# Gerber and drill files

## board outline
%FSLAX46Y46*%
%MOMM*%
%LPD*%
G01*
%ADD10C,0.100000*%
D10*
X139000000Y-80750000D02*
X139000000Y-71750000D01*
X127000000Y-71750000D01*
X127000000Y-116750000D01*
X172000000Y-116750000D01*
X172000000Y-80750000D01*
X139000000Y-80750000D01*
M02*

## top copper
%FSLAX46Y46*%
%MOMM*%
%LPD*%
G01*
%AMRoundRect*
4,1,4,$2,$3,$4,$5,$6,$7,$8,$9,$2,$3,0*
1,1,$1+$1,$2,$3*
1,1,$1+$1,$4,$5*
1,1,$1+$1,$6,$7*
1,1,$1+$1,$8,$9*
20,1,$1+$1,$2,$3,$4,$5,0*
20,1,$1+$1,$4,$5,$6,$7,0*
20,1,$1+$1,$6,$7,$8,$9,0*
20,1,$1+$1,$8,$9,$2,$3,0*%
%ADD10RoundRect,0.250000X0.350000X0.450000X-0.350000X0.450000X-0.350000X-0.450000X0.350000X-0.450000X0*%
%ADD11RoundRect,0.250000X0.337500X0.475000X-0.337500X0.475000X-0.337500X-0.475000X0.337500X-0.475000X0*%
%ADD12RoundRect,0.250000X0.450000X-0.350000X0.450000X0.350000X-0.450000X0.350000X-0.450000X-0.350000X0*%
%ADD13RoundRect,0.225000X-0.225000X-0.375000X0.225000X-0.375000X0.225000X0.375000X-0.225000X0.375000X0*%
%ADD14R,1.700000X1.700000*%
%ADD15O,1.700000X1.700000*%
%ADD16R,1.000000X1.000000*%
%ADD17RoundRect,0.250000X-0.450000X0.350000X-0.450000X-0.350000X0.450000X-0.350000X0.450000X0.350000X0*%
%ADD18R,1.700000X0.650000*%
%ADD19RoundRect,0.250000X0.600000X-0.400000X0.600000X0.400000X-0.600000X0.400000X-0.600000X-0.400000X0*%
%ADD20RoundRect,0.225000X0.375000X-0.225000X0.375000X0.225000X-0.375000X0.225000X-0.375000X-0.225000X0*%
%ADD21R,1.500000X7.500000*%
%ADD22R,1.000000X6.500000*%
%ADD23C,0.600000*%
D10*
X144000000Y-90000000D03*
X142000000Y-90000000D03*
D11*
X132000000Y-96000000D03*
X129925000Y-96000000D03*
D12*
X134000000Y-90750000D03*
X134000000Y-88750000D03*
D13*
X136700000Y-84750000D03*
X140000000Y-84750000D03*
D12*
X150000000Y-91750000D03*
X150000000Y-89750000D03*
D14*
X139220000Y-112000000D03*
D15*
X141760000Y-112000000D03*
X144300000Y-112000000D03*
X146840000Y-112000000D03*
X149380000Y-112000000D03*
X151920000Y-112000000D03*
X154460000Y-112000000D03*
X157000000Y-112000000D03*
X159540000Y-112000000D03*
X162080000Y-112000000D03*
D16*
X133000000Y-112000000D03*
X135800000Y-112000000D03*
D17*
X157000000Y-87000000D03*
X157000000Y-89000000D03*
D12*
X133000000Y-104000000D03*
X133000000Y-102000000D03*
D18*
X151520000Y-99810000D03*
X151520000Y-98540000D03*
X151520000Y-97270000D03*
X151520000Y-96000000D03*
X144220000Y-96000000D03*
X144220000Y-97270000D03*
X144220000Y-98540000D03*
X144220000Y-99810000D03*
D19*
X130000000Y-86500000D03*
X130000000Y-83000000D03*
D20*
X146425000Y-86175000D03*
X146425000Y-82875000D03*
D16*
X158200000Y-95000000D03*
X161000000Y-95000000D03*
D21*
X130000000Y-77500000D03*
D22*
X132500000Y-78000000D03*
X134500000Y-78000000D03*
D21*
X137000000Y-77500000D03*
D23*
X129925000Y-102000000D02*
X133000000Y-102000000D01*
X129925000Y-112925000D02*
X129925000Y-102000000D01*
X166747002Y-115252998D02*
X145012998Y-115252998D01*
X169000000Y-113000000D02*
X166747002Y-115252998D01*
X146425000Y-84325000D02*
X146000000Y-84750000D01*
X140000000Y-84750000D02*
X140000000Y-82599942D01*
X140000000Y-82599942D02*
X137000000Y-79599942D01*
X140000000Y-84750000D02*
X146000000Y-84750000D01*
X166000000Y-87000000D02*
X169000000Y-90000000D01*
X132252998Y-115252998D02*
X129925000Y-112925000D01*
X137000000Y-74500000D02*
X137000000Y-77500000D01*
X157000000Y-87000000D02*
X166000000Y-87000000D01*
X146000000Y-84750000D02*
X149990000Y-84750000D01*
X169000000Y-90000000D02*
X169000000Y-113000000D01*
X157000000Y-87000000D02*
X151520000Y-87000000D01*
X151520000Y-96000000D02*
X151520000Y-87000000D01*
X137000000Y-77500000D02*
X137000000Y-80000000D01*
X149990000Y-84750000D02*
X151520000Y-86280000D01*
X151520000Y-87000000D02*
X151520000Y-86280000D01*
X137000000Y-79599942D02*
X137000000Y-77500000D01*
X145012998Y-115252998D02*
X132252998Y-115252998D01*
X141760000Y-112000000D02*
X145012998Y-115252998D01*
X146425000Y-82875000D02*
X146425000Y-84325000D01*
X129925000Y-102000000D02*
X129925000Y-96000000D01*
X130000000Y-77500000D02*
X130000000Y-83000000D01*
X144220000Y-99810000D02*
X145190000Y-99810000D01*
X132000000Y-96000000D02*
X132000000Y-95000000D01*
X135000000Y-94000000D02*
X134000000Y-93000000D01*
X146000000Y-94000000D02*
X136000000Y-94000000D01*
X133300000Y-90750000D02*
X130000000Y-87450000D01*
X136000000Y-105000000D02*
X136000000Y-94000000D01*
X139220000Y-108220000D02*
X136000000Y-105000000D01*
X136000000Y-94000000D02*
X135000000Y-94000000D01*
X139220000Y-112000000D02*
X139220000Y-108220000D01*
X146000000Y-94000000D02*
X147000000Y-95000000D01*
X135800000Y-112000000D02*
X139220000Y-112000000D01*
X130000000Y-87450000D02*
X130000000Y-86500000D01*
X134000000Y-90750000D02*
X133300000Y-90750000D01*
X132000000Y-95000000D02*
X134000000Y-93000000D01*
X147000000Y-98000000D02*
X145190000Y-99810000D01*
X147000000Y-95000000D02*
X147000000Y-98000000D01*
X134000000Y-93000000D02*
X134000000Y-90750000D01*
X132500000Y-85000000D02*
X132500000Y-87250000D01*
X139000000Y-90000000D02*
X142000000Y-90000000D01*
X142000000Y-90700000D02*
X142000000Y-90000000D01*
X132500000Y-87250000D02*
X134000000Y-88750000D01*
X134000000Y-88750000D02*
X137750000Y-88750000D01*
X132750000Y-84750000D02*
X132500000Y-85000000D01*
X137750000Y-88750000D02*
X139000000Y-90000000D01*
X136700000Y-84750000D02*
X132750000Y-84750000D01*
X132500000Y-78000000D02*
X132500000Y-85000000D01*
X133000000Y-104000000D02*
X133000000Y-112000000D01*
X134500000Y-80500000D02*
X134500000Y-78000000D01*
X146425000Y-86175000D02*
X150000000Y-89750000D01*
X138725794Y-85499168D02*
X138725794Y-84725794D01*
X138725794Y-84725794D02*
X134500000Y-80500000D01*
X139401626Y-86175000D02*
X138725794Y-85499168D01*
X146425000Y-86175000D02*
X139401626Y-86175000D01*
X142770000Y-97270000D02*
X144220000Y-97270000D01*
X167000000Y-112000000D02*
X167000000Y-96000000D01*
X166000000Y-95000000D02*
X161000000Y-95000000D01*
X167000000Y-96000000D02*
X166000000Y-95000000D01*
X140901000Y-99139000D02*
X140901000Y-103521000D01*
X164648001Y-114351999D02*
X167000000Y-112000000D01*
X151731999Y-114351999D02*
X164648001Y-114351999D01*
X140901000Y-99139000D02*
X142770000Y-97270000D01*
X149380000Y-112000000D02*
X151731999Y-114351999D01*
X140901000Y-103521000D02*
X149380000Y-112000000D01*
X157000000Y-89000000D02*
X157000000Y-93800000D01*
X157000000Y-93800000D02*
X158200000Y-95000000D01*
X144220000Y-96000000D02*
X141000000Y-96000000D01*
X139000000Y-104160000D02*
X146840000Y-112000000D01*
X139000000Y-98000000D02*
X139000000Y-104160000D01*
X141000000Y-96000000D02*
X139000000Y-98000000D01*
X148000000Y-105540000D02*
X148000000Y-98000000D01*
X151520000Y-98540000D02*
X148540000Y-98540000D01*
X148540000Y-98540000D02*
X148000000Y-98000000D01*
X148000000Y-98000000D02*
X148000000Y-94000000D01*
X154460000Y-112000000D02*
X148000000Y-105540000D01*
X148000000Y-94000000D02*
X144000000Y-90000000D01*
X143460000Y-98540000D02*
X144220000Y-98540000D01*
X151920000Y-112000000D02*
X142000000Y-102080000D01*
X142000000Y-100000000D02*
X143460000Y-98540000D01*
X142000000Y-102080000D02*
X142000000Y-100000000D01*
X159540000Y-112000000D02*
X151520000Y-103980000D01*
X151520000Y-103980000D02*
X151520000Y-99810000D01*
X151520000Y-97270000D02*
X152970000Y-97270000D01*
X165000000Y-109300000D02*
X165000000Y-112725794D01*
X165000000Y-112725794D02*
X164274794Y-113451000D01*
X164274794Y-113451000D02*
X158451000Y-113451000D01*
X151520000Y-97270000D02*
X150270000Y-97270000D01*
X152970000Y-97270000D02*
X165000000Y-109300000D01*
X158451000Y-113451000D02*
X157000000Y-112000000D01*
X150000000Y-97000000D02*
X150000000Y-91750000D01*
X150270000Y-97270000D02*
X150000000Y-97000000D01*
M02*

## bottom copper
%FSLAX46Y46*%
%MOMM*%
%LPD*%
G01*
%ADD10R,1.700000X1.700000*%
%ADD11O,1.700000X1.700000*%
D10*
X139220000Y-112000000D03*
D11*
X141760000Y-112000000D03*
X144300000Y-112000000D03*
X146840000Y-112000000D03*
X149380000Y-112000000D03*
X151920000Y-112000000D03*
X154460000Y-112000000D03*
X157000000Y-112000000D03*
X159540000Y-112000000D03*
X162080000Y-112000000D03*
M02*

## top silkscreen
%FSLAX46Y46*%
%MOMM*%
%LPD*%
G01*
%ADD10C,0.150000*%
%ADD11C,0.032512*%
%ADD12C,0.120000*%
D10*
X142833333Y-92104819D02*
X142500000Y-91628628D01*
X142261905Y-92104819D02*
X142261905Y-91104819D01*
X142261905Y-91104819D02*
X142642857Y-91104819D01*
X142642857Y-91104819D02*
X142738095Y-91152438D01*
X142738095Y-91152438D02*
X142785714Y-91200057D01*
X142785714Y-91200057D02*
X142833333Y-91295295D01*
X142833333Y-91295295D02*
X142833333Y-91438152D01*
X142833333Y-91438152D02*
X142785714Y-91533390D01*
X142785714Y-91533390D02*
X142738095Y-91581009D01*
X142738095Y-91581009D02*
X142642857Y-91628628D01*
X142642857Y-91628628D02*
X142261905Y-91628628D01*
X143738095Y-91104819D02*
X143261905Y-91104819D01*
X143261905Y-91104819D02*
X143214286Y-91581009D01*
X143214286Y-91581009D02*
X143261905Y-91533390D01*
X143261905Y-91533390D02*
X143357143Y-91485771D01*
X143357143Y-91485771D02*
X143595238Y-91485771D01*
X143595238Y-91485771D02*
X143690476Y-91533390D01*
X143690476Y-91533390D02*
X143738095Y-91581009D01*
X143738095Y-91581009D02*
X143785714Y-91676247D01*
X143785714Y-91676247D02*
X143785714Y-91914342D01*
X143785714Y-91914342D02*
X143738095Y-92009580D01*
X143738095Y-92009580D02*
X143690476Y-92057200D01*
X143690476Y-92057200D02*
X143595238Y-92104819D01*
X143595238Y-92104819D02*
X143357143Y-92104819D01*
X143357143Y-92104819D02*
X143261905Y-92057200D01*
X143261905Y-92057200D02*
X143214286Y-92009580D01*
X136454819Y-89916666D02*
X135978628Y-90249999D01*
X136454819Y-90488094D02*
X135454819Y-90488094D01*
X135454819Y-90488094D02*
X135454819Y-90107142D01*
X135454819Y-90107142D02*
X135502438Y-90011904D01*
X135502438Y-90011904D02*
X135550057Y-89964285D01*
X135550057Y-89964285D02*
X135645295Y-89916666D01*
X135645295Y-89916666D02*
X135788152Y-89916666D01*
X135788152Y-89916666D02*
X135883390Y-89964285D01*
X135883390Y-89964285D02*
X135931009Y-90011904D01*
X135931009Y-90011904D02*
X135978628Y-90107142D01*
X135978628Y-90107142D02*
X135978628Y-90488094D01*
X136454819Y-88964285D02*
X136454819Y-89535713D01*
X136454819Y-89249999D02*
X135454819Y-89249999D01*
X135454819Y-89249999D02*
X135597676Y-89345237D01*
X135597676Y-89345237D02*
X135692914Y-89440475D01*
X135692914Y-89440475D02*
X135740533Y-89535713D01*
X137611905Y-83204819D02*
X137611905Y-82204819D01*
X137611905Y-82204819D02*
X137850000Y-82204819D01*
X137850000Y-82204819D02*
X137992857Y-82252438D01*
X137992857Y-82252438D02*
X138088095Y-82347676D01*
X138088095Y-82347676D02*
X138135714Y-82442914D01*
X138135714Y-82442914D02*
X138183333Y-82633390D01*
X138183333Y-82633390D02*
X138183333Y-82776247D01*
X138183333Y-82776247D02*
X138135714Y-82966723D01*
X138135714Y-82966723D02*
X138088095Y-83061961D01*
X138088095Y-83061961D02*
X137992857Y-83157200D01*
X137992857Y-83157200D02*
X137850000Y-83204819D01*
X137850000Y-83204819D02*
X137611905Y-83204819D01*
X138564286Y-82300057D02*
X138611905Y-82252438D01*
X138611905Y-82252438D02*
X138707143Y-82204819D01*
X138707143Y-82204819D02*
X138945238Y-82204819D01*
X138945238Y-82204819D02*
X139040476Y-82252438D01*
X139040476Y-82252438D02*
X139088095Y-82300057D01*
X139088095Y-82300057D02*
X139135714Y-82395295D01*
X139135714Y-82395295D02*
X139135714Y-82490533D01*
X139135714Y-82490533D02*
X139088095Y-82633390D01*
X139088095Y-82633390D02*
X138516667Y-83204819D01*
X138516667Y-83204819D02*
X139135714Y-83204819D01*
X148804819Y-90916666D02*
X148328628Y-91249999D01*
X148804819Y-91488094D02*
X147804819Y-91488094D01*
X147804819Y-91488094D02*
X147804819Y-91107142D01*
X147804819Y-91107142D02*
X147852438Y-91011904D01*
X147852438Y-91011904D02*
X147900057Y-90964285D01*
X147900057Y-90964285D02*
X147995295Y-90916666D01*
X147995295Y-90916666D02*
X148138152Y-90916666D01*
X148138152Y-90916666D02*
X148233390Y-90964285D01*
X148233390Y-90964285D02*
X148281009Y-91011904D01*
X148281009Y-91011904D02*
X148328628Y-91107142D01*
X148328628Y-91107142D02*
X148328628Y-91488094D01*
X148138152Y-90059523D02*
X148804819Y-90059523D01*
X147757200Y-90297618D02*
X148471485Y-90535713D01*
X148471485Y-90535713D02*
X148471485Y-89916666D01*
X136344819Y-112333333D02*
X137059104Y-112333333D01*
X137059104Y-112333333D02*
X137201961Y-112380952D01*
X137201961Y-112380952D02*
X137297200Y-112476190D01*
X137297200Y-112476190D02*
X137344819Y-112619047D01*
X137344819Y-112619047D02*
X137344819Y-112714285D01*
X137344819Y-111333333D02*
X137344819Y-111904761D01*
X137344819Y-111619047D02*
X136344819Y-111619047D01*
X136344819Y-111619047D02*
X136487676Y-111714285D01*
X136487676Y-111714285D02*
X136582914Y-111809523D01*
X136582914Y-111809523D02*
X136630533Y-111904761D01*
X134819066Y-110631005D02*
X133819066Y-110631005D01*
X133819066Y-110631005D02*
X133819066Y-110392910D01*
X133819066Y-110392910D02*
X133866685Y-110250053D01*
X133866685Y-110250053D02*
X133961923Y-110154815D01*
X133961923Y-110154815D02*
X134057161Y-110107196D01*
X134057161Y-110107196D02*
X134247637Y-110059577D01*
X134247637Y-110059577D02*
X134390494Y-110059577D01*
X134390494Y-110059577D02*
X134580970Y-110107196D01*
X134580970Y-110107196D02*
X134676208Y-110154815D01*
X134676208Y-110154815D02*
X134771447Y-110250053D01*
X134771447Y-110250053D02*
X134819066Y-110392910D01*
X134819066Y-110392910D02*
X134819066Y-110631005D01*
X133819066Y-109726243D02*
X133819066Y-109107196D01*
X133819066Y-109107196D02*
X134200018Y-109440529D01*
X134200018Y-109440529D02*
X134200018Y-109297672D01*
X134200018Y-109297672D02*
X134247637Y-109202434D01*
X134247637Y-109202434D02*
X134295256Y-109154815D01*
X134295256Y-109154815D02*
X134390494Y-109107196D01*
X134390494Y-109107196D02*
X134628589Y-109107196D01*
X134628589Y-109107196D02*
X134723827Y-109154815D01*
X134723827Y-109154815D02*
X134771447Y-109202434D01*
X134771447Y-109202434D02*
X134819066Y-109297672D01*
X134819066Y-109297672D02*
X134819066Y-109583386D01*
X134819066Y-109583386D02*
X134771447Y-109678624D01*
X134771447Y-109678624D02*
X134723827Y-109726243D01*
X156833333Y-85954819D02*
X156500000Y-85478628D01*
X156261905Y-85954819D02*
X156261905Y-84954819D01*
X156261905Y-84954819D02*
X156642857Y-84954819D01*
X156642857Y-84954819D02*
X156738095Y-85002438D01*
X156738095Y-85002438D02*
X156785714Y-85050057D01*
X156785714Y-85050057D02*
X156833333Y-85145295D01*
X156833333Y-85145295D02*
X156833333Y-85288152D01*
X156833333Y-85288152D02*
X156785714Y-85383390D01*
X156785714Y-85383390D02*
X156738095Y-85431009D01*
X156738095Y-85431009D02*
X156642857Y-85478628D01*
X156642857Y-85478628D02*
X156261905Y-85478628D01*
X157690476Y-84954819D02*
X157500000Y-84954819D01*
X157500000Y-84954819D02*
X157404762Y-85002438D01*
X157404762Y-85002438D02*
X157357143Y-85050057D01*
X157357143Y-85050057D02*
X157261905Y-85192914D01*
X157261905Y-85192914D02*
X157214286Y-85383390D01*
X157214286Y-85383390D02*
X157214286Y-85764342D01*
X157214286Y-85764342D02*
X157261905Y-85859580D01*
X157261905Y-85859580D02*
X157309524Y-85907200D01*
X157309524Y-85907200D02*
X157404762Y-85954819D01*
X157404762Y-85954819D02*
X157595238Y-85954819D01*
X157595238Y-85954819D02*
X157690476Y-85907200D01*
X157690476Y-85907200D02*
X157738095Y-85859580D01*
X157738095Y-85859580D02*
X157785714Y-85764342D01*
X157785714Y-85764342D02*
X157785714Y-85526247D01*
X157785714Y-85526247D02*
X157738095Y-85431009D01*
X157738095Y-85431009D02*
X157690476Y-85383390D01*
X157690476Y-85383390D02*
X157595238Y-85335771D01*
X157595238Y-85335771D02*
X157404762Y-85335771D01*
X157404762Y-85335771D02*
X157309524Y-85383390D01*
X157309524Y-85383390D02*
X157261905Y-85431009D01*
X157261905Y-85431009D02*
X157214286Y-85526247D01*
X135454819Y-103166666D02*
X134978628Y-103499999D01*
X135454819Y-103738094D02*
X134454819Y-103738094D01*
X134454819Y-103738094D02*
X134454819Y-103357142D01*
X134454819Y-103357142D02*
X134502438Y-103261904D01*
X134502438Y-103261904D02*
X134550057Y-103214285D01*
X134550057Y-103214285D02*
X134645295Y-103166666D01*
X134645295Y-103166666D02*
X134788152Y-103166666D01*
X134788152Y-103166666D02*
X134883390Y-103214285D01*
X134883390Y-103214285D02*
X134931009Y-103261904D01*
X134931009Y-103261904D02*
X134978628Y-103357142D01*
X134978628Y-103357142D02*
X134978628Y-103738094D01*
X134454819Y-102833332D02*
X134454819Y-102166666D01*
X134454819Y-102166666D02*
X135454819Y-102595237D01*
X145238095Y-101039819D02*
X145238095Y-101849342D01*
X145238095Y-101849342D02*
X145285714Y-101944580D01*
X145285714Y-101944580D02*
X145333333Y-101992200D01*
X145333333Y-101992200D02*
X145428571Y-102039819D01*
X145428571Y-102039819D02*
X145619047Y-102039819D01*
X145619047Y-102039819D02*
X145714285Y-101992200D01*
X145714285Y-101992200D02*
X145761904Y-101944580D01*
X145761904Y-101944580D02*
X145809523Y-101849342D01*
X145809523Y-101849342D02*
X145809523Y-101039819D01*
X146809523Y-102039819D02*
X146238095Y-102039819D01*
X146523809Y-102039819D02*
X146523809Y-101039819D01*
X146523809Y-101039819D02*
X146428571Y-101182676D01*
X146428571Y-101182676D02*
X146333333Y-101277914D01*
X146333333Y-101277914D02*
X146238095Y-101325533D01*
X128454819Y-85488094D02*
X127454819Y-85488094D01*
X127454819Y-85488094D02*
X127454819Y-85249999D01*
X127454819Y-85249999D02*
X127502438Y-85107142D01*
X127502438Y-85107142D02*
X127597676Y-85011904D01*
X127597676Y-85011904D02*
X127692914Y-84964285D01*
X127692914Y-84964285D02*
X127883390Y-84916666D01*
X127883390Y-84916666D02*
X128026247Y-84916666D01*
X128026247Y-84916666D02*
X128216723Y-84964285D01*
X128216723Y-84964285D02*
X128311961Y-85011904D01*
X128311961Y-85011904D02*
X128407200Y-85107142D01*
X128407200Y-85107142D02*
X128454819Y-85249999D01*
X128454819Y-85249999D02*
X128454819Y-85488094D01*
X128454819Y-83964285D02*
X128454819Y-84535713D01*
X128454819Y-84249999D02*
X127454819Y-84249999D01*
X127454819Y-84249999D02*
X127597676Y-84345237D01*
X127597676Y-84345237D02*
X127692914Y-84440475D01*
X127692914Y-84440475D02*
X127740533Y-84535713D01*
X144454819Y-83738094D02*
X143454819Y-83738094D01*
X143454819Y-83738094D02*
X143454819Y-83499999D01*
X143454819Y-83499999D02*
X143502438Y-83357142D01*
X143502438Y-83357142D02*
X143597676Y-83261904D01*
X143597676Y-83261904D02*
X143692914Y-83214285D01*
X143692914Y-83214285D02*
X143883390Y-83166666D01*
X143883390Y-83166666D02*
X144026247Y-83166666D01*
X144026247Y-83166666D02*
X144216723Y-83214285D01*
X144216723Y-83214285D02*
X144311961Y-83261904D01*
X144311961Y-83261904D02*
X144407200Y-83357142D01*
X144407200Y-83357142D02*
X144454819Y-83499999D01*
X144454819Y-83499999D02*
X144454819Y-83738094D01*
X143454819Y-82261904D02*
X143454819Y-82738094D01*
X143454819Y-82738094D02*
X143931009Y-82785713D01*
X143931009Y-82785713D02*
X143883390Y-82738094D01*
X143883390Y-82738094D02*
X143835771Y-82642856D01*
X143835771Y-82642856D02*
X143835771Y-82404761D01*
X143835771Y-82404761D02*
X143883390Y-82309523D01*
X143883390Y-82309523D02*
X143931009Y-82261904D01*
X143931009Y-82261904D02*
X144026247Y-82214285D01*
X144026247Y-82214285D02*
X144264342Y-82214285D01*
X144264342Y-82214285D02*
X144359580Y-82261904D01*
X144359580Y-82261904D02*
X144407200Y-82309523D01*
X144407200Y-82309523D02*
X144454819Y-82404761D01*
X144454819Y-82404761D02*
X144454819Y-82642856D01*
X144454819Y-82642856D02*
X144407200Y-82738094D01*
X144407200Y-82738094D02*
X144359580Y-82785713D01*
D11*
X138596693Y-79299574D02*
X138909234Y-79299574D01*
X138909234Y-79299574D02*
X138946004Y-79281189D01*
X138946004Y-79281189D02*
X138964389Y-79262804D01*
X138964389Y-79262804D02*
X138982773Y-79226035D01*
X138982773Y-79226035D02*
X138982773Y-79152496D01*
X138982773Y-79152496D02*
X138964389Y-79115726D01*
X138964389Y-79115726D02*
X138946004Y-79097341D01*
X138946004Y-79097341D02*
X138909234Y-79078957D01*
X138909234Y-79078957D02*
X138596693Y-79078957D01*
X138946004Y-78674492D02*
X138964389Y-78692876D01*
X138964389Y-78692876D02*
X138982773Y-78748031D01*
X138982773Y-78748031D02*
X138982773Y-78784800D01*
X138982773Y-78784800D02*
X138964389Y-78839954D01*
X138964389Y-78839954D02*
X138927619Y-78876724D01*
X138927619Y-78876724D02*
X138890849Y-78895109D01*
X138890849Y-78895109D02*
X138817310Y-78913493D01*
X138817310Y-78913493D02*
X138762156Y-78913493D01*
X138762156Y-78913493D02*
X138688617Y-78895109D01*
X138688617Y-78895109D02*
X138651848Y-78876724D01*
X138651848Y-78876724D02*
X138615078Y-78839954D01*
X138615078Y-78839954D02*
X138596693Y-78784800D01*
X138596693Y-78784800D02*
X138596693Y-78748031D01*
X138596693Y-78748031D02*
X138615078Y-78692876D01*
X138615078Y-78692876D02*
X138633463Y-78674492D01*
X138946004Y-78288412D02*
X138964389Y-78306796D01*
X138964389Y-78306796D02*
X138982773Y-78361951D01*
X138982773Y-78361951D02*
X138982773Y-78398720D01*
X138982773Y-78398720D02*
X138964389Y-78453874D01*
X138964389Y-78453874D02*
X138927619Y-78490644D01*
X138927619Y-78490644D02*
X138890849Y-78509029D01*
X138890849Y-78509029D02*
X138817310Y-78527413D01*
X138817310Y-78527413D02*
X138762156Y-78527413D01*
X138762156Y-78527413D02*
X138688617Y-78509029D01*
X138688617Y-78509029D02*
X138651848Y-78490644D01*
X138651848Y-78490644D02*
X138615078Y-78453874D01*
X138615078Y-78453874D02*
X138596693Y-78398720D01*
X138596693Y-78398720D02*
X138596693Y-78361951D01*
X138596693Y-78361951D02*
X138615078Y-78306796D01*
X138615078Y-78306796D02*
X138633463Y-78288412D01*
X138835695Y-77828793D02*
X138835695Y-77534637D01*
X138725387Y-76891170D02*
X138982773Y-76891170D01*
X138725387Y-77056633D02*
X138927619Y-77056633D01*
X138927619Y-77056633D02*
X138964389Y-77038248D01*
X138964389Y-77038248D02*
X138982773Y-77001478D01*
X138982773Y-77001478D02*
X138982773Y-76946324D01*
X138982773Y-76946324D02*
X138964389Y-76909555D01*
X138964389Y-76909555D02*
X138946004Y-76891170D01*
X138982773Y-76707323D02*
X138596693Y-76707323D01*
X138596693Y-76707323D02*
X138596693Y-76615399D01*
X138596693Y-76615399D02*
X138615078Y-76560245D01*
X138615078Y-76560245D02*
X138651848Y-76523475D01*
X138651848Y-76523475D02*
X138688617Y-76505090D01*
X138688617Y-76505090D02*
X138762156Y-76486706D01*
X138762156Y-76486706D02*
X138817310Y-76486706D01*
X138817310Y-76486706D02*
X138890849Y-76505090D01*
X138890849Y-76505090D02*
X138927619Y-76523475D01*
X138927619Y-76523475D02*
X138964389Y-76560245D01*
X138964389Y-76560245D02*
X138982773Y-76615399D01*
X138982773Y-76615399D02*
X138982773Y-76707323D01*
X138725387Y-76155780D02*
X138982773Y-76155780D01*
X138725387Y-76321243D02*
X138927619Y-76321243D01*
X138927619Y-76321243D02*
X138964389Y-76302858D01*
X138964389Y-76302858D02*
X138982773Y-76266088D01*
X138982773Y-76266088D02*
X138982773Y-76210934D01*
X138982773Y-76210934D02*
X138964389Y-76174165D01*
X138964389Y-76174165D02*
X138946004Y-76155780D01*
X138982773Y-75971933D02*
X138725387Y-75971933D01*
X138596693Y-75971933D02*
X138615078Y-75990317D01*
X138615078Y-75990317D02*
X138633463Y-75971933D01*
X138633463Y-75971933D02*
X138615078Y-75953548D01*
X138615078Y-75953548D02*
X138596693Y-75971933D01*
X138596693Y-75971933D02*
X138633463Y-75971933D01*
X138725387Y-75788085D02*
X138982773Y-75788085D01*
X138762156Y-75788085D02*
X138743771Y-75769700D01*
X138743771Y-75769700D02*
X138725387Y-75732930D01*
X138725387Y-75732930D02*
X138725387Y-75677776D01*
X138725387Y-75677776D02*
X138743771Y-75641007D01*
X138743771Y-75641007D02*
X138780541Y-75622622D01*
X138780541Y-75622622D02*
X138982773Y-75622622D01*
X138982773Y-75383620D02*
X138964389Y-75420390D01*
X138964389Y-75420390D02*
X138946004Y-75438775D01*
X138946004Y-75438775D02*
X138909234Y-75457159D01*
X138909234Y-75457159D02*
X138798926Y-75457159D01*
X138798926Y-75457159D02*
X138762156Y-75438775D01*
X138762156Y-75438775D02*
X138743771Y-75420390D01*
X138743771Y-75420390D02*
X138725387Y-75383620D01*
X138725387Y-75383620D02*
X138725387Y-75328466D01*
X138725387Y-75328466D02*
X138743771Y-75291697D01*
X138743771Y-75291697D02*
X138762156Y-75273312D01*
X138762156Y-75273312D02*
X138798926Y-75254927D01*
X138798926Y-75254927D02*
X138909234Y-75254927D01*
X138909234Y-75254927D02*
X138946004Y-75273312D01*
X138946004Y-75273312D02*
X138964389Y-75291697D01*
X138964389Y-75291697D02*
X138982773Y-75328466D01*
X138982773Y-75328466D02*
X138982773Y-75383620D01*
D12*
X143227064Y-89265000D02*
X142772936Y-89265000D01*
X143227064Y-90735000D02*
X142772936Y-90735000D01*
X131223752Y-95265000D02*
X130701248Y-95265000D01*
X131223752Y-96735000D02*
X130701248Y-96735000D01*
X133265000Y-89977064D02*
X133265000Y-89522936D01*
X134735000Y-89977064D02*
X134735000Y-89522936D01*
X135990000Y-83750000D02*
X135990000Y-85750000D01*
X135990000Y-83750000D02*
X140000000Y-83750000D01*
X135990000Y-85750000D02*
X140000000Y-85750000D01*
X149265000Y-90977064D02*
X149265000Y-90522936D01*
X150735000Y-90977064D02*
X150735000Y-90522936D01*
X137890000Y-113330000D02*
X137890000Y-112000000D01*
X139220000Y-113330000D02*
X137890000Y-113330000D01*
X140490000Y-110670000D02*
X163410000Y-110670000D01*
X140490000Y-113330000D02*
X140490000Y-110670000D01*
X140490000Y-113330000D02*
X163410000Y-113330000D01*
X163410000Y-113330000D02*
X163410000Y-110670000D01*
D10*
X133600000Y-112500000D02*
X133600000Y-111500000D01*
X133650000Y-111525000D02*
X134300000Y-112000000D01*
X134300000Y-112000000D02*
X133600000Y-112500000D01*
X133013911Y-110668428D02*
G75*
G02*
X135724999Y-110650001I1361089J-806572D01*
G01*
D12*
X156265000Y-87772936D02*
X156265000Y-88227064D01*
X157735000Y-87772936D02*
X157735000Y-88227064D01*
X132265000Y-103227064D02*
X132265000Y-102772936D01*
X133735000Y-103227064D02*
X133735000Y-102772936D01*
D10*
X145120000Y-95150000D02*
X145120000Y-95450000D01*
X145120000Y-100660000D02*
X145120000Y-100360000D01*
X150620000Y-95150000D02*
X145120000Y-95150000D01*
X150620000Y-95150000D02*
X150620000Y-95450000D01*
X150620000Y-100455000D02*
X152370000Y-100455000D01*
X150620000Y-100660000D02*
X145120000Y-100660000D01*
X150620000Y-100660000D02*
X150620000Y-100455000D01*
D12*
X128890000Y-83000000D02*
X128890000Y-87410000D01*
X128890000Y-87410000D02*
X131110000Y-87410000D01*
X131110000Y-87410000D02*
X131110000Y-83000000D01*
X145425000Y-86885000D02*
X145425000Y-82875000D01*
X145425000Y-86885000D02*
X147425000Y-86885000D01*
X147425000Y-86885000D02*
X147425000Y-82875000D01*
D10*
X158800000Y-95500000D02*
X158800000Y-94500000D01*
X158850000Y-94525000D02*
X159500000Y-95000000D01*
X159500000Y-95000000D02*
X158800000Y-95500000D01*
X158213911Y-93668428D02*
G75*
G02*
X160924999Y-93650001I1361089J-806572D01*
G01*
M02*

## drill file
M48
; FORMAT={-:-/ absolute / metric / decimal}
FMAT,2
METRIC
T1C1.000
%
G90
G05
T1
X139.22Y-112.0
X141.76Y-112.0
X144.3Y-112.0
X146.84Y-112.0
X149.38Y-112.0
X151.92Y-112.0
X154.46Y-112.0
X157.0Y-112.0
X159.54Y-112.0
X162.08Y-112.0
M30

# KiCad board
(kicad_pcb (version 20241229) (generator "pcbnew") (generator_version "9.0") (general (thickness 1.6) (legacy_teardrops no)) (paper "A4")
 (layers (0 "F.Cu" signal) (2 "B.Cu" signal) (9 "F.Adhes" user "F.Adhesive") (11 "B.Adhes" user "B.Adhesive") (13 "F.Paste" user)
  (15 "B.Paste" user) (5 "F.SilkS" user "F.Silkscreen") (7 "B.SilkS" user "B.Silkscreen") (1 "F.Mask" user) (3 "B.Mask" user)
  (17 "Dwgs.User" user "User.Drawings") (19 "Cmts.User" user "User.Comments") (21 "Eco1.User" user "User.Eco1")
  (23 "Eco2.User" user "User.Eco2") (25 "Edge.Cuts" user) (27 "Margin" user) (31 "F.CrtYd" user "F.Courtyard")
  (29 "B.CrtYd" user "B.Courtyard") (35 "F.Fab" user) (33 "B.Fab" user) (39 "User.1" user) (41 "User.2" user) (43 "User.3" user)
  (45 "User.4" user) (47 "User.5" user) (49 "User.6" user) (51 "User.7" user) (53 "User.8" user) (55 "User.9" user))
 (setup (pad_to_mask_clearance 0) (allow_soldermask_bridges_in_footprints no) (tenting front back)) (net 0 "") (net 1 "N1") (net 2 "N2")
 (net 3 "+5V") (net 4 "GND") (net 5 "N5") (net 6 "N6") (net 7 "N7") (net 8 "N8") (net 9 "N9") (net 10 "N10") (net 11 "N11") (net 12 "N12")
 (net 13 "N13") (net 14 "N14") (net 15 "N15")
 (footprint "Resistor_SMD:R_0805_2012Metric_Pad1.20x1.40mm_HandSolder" (layer "F.Cu") (at 143 90 180)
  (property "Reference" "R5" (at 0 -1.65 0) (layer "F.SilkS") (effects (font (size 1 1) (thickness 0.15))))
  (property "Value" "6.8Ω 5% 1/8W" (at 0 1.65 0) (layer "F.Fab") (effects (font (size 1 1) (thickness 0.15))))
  (fp_line (start -0.227064 0.735) (end 0.227064 0.735) (stroke (width 0.12) (type solid)) (layer "F.SilkS"))
  (fp_line (start -0.227064 -0.735) (end 0.227064 -0.735) (stroke (width 0.12) (type solid)) (layer "F.SilkS"))
  (pad "1" smd roundrect (at -1 0 180) (size 1.2 1.4) (layers "F.Cu" "F.Mask" "F.Paste") (roundrect_rratio 0.208333) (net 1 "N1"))
  (pad "2" smd roundrect (at 1 0 180) (size 1.2 1.4) (layers "F.Cu" "F.Mask" "F.Paste") (roundrect_rratio 0.208333) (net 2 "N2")))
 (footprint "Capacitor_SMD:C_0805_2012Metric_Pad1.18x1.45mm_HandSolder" (layer "F.Cu") (at 130.9625 96 180)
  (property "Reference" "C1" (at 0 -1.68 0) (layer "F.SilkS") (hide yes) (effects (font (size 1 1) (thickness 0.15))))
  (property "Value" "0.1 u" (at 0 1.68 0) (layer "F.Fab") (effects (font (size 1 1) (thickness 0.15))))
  (fp_line (start -0.261252 0.735) (end 0.261252 0.735) (stroke (width 0.12) (type solid)) (layer "F.SilkS"))
  (fp_line (start -0.261252 -0.735) (end 0.261252 -0.735) (stroke (width 0.12) (type solid)) (layer "F.SilkS"))
  (pad "1" smd roundrect (at -1.0375 0 180) (size 1.175 1.45) (layers "F.Cu" "F.Mask" "F.Paste") (roundrect_rratio 0.212766) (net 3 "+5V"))
  (pad "2" smd roundrect (at 1.0375 0 180) (size 1.175 1.45) (layers "F.Cu" "F.Mask" "F.Paste") (roundrect_rratio 0.212766) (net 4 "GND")))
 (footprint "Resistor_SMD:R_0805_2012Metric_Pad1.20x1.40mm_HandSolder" (layer "F.Cu") (at 134 89.75 90)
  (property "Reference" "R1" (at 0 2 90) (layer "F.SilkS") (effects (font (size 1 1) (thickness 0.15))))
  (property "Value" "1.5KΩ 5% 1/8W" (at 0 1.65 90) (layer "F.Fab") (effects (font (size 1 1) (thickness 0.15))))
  (fp_line (start -0.227064 -0.735) (end 0.227064 -0.735) (stroke (width 0.12) (type solid)) (layer "F.SilkS"))
  (fp_line (start -0.227064 0.735) (end 0.227064 0.735) (stroke (width 0.12) (type solid)) (layer "F.SilkS"))
  (pad "1" smd roundrect (at -1 0 90) (size 1.2 1.4) (layers "F.Cu" "F.Mask" "F.Paste") (roundrect_rratio 0.208333) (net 3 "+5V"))
  (pad "2" smd roundrect (at 1 0 90) (size 1.2 1.4) (layers "F.Cu" "F.Mask" "F.Paste") (roundrect_rratio 0.208333) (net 2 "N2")))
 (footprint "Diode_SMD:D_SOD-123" (layer "F.Cu") (at 138.35 84.75)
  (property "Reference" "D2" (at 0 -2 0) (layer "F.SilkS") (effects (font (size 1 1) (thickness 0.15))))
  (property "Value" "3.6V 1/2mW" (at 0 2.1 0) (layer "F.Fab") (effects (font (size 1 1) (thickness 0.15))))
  (fp_line (start -2.36 -1) (end -2.36 1) (stroke (width 0.12) (type solid)) (layer "F.SilkS"))
  (fp_line (start -2.36 -1) (end 1.65 -1) (stroke (width 0.12) (type solid)) (layer "F.SilkS"))
  (fp_line (start -2.36 1) (end 1.65 1) (stroke (width 0.12) (type solid)) (layer "F.SilkS"))
  (pad "1" smd roundrect (at -1.65 0) (size 0.9 1.2) (layers "F.Cu" "F.Mask" "F.Paste") (roundrect_rratio 0.25) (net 2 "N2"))
  (pad "2" smd roundrect (at 1.65 0) (size 0.9 1.2) (layers "F.Cu" "F.Mask" "F.Paste") (roundrect_rratio 0.25) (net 4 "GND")))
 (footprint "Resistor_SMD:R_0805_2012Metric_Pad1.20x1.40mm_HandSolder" (layer "F.Cu") (at 150 90.75 90)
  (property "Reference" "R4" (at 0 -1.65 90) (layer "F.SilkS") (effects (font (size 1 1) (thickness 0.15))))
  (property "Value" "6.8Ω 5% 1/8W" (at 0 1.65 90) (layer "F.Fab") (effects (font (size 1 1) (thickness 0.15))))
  (fp_line (start -0.227064 -0.735) (end 0.227064 -0.735) (stroke (width 0.12) (type solid)) (layer "F.SilkS"))
  (fp_line (start -0.227064 0.735) (end 0.227064 0.735) (stroke (width 0.12) (type solid)) (layer "F.SilkS"))
  (pad "1" smd roundrect (at -1 0 90) (size 1.2 1.4) (layers "F.Cu" "F.Mask" "F.Paste") (roundrect_rratio 0.208333) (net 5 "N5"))
  (pad "2" smd roundrect (at 1 0 90) (size 1.2 1.4) (layers "F.Cu" "F.Mask" "F.Paste") (roundrect_rratio 0.208333) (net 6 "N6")))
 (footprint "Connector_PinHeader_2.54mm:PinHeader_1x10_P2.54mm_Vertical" (layer "F.Cu") (at 139.22 112 90)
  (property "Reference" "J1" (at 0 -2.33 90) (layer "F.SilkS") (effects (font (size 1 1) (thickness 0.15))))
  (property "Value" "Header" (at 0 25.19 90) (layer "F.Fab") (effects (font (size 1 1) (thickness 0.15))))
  (fp_line (start -1.33 -1.33) (end 0 -1.33) (stroke (width 0.12) (type solid)) (layer "F.SilkS"))
  (fp_line (start -1.33 0) (end -1.33 -1.33) (stroke (width 0.12) (type solid)) (layer "F.SilkS"))
  (fp_line (start 1.33 1.27) (end 1.33 24.19) (stroke (width 0.12) (type solid)) (layer "F.SilkS"))
  (fp_line (start -1.33 1.27) (end 1.33 1.27) (stroke (width 0.12) (type solid)) (layer "F.SilkS"))
  (fp_line (start -1.33 1.27) (end -1.33 24.19) (stroke (width 0.12) (type solid)) (layer "F.SilkS"))
  (fp_line (start -1.33 24.19) (end 1.33 24.19) (stroke (width 0.12) (type solid)) (layer "F.SilkS"))
  (pad "1" thru_hole rect (at 0 0 90) (size 1.7 1.7) (drill 1) (layers "*.Cu" "*.Mask") (remove_unused_layers no) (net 3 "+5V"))
  (pad "2" thru_hole oval (at 0 2.54 90) (size 1.7 1.7) (drill 1) (layers "*.Cu" "*.Mask") (remove_unused_layers no) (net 4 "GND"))
  (pad "3" thru_hole oval (at 0 5.08 90) (size 1.7 1.7) (drill 1) (layers "*.Cu" "*.Mask") (remove_unused_layers no) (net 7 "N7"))
  (pad "4" thru_hole oval (at 0 7.62 90) (size 1.7 1.7) (drill 1) (layers "*.Cu" "*.Mask") (remove_unused_layers no) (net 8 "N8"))
  (pad "5" thru_hole oval (at 0 10.16 90) (size 1.7 1.7) (drill 1) (layers "*.Cu" "*.Mask") (remove_unused_layers no) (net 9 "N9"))
  (pad "6" thru_hole oval (at 0 12.7 90) (size 1.7 1.7) (drill 1) (layers "*.Cu" "*.Mask") (remove_unused_layers no) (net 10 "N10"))
  (pad "7" thru_hole oval (at 0 15.24 90) (size 1.7 1.7) (drill 1) (layers "*.Cu" "*.Mask") (remove_unused_layers no) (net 1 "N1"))
  (pad "8" thru_hole oval (at 0 17.78 90) (size 1.7 1.7) (drill 1) (layers "*.Cu" "*.Mask") (remove_unused_layers no) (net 5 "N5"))
  (pad "9" thru_hole oval (at 0 20.32 90) (size 1.7 1.7) (drill 1) (layers "*.Cu" "*.Mask") (remove_unused_layers no) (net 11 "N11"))
  (pad "10" thru_hole oval (at 0 22.86 90) (size 1.7 1.7) (drill 1) (layers "*.Cu" "*.Mask") (remove_unused_layers no) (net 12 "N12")))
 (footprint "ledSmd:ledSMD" (layer "F.Cu") (at 134.8 112)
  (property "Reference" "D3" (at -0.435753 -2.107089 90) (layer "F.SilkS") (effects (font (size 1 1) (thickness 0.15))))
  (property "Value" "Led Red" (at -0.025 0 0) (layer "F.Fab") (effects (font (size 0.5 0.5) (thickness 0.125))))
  (fp_line (start -1.2 0.5) (end -1.2 -0.5) (stroke (width 0.15) (type solid)) (layer "F.SilkS"))
  (fp_line (start -1.15 -0.475) (end -0.5 0) (stroke (width 0.15) (type solid)) (layer "F.SilkS"))
  (fp_line (start -0.5 0) (end -1.2 0.5) (stroke (width 0.15) (type solid)) (layer "F.SilkS"))
  (fp_arc (start -1.786089 -1.331572) (mid -0.435753 -2.107089) (end 0.924999 -1.349999) (stroke (width 0.15) (type solid))
   (layer "F.SilkS"))
  (pad "1" smd rect (at -1.8 0) (size 1 1) (layers "F.Cu" "F.Mask" "F.Paste") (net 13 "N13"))
  (pad "2" smd rect (at 1 0) (size 1 1) (layers "F.Cu" "F.Mask" "F.Paste") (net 3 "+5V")))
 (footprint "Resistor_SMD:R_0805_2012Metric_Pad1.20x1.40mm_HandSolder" (layer "F.Cu") (at 157 88 -90)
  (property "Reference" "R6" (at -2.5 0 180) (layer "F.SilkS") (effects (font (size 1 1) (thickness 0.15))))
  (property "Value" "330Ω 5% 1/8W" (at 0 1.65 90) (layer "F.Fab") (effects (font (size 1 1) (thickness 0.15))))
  (fp_line (start -0.227064 0.735) (end 0.227064 0.735) (stroke (width 0.12) (type solid)) (layer "F.SilkS"))
  (fp_line (start -0.227064 -0.735) (end 0.227064 -0.735) (stroke (width 0.12) (type solid)) (layer "F.SilkS"))
  (pad "1" smd roundrect (at -1 0 270) (size 1.2 1.4) (layers "F.Cu" "F.Mask" "F.Paste") (roundrect_rratio 0.208333) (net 4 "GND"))
  (pad "2" smd roundrect (at 1 0 270) (size 1.2 1.4) (layers "F.Cu" "F.Mask" "F.Paste") (roundrect_rratio 0.208333) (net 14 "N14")))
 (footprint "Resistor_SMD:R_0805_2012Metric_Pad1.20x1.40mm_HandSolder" (layer "F.Cu") (at 133 103 90)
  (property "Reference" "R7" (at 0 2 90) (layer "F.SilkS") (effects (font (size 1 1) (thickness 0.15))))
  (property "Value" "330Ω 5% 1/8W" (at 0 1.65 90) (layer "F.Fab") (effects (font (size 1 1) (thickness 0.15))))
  (fp_line (start -0.227064 -0.735) (end 0.227064 -0.735) (stroke (width 0.12) (type solid)) (layer "F.SilkS"))
  (fp_line (start -0.227064 0.735) (end 0.227064 0.735) (stroke (width 0.12) (type solid)) (layer "F.SilkS"))
  (pad "1" smd roundrect (at -1 0 90) (size 1.2 1.4) (layers "F.Cu" "F.Mask" "F.Paste") (roundrect_rratio 0.208333) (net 13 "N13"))
  (pad "2" smd roundrect (at 1 0 90) (size 1.2 1.4) (layers "F.Cu" "F.Mask" "F.Paste") (roundrect_rratio 0.208333) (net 4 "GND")))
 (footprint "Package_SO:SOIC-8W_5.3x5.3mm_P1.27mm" (layer "F.Cu") (at 147.87 97.905 180)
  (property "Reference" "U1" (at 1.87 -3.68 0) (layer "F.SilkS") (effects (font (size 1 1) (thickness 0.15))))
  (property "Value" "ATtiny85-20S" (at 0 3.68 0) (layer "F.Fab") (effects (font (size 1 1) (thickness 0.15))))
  (fp_line (start 2.75 2.755) (end 2.75 2.455) (stroke (width 0.15) (type solid)) (layer "F.SilkS"))
  (fp_line (start 2.75 -2.755) (end 2.75 -2.455) (stroke (width 0.15) (type solid)) (layer "F.SilkS"))
  (fp_line (start -2.75 2.755) (end 2.75 2.755) (stroke (width 0.15) (type solid)) (layer "F.SilkS"))
  (fp_line (start -2.75 2.755) (end -2.75 2.455) (stroke (width 0.15) (type solid)) (layer "F.SilkS"))
  (fp_line (start -2.75 -2.55) (end -4.5 -2.55) (stroke (width 0.15) (type solid)) (layer "F.SilkS"))
  (fp_line (start -2.75 -2.755) (end 2.75 -2.755) (stroke (width 0.15) (type solid)) (layer "F.SilkS"))
  (fp_line (start -2.75 -2.755) (end -2.75 -2.55) (stroke (width 0.15) (type solid)) (layer "F.SilkS"))
  (pad "1" smd rect (at -3.65 -1.905 180) (size 1.7 0.65) (layers "F.Cu" "F.Mask" "F.Paste") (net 11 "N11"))
  (pad "2" smd rect (at -3.65 -0.635 180) (size 1.7 0.65) (layers "F.Cu" "F.Mask" "F.Paste") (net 1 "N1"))
  (pad "3" smd rect (at -3.65 0.635 180) (size 1.7 0.65) (layers "F.Cu" "F.Mask" "F.Paste") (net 5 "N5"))
  (pad "4" smd rect (at -3.65 1.905 180) (size 1.7 0.65) (layers "F.Cu" "F.Mask" "F.Paste") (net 4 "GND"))
  (pad "5" smd rect (at 3.65 1.905 180) (size 1.7 0.65) (layers "F.Cu" "F.Mask" "F.Paste") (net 8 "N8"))
  (pad "6" smd rect (at 3.65 0.635 180) (size 1.7 0.65) (layers "F.Cu" "F.Mask" "F.Paste") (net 9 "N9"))
  (pad "7" smd rect (at 3.65 -0.635 180) (size 1.7 0.65) (layers "F.Cu" "F.Mask" "F.Paste") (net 10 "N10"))
  (pad "8" smd rect (at 3.65 -1.905 180) (size 1.7 0.65) (layers "F.Cu" "F.Mask" "F.Paste") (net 3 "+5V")))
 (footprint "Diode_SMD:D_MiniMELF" (layer "F.Cu") (at 130 84.75 90)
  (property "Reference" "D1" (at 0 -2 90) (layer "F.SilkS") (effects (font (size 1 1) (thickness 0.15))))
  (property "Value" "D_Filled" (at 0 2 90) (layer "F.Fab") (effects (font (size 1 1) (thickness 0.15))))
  (fp_line (start 1.75 -1.11) (end -2.66 -1.11) (stroke (width 0.12) (type solid)) (layer "F.SilkS"))
  (fp_line (start -2.66 -1.11) (end -2.66 1.11) (stroke (width 0.12) (type solid)) (layer "F.SilkS"))
  (fp_line (start -2.66 1.11) (end 1.75 1.11) (stroke (width 0.12) (type solid)) (layer "F.SilkS"))
  (pad "1" smd roundrect (at -1.75 0 90) (size 1.3 1.7) (layers "F.Cu" "F.Mask" "F.Paste") (roundrect_rratio 0.1923076923) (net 3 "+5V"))
  (pad "2" smd roundrect (at 1.75 0 90) (size 1.3 1.7) (layers "F.Cu" "F.Mask" "F.Paste") (roundrect_rratio 0.1923076923) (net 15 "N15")))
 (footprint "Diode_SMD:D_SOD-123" (layer "F.Cu") (at 146.425 84.525 90)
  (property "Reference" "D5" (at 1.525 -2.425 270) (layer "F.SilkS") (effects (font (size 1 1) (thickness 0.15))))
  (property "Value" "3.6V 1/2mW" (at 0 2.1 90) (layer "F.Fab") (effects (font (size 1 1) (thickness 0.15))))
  (fp_line (start -2.36 -1) (end 1.65 -1) (stroke (width 0.12) (type solid)) (layer "F.SilkS"))
  (fp_line (start -2.36 -1) (end -2.36 1) (stroke (width 0.12) (type solid)) (layer "F.SilkS"))
  (fp_line (start -2.36 1) (end 1.65 1) (stroke (width 0.12) (type solid)) (layer "F.SilkS"))
  (pad "1" smd roundrect (at -1.65 0 90) (size 0.9 1.2) (layers "F.Cu" "F.Mask" "F.Paste") (roundrect_rratio 0.25) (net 6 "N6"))
  (pad "2" smd roundrect (at 1.65 0 90) (size 0.9 1.2) (layers "F.Cu" "F.Mask" "F.Paste") (roundrect_rratio 0.25) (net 4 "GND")))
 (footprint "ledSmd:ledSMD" (layer "F.Cu") (at 160 95)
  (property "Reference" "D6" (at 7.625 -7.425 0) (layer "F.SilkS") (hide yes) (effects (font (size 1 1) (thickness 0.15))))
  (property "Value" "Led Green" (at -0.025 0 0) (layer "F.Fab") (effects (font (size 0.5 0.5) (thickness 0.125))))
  (fp_line (start -1.2 0.5) (end -1.2 -0.5) (stroke (width 0.15) (type solid)) (layer "F.SilkS"))
  (fp_line (start -1.15 -0.475) (end -0.5 0) (stroke (width 0.15) (type solid)) (layer "F.SilkS"))
  (fp_line (start -0.5 0) (end -1.2 0.5) (stroke (width 0.15) (type solid)) (layer "F.SilkS"))
  (fp_arc (start -1.786089 -1.331572) (mid -0.435753 -2.107089) (end 0.924999 -1.349999) (stroke (width 0.15) (type solid))
   (layer "F.SilkS"))
  (pad "1" smd rect (at -1.8 0) (size 1 1) (layers "F.Cu" "F.Mask" "F.Paste") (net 14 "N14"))
  (pad "2" smd rect (at 1 0) (size 1 1) (layers "F.Cu" "F.Mask" "F.Paste") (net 9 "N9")))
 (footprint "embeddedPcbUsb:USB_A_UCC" (layer "F.Cu") (at 133.5 77.7 -90)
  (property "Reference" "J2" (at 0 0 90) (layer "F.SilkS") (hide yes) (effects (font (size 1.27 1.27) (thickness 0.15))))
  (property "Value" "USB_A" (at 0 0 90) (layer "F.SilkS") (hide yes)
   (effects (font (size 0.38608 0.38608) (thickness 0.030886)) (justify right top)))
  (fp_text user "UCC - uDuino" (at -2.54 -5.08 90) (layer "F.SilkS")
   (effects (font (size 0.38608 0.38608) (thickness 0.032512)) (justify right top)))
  (pad "1" smd rect (at -0.2 3.5 270) (size 7.5 1.5) (layers "F.Cu" "F.Mask" "F.Paste") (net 15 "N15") (solder_mask_margin 0.1016))
  (pad "2" smd rect (at 0.3 1 270) (size 6.5 1) (layers "F.Cu" "F.Mask" "F.Paste") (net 2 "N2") (solder_mask_margin 0.1016))
  (pad "3" smd rect (at 0.3 -1 270) (size 6.5 1) (layers "F.Cu" "F.Mask" "F.Paste") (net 6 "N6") (solder_mask_margin 0.1016))
  (pad "4" smd rect (at -0.2 -3.5 270) (size 7.5 1.5) (layers "F.Cu" "F.Mask" "F.Paste") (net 4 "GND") (solder_mask_margin 0.1016)))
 (gr_poly
  (pts (xy 139 80.75) (xy 139 71.75) (xy 127 71.75) (xy 127 116.75) (xy 172 116.75) (xy 172 80.75)) (stroke (width 0.1) (type solid))
  (fill no) (layer "Edge.Cuts"))
 (segment (start 129.925 102) (end 133 102) (width 0.6) (layer "F.Cu") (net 4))
 (segment (start 129.925 112.925) (end 129.925 102) (width 0.6) (layer "F.Cu") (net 4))
 (segment (start 166.747002 115.252998) (end 145.012998 115.252998) (width 0.6) (layer "F.Cu") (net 4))
 (segment (start 169 113) (end 166.747002 115.252998) (width 0.6) (layer "F.Cu") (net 4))
 (segment (start 146.425 84.325) (end 146 84.75) (width 0.6) (layer "F.Cu") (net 4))
 (segment (start 140 84.75) (end 140 82.599942) (width 0.6) (layer "F.Cu") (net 4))
 (segment (start 140 82.599942) (end 137 79.599942) (width 0.6) (layer "F.Cu") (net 4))
 (segment (start 140 84.75) (end 146 84.75) (width 0.6) (layer "F.Cu") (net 4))
 (segment (start 166 87) (end 169 90) (width 0.6) (layer "F.Cu") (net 4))
 (segment (start 132.252998 115.252998) (end 129.925 112.925) (width 0.6) (layer "F.Cu") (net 4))
 (segment (start 137 74.5) (end 137 77.5) (width 0.6) (layer "F.Cu") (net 4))
 (segment (start 157 87) (end 166 87) (width 0.6) (layer "F.Cu") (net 4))
 (segment (start 146 84.75) (end 149.99 84.75) (width 0.6) (layer "F.Cu") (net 4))
 (segment (start 169 90) (end 169 113) (width 0.6) (layer "F.Cu") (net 4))
 (segment (start 157 87) (end 151.52 87) (width 0.6) (layer "F.Cu") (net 4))
 (segment (start 151.52 96) (end 151.52 87) (width 0.6) (layer "F.Cu") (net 4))
 (segment (start 137 77.5) (end 137 80) (width 0.6) (layer "F.Cu") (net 4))
 (segment (start 149.99 84.75) (end 151.52 86.28) (width 0.6) (layer "F.Cu") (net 4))
 (segment (start 151.52 87) (end 151.52 86.28) (width 0.6) (layer "F.Cu") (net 4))
 (segment (start 137 79.599942) (end 137 77.5) (width 0.6) (layer "F.Cu") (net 4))
 (segment (start 145.012998 115.252998) (end 132.252998 115.252998) (width 0.6) (layer "F.Cu") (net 4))
 (segment (start 141.76 112) (end 145.012998 115.252998) (width 0.6) (layer "F.Cu") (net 4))
 (segment (start 146.425 82.875) (end 146.425 84.325) (width 0.6) (layer "F.Cu") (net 4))
 (segment (start 129.925 102) (end 129.925 96) (width 0.6) (layer "F.Cu") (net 4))
 (segment (start 130 77.5) (end 130 83) (width 0.6) (layer "F.Cu") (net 15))
 (segment (start 144.22 99.81) (end 145.19 99.81) (width 0.6) (layer "F.Cu") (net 3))
 (segment (start 132 96) (end 132 95) (width 0.6) (layer "F.Cu") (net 3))
 (segment (start 135 94) (end 134 93) (width 0.6) (layer "F.Cu") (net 3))
 (segment (start 146 94) (end 136 94) (width 0.6) (layer "F.Cu") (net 3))
 (segment (start 133.3 90.75) (end 130 87.45) (width 0.6) (layer "F.Cu") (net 3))
 (segment (start 136 105) (end 136 94) (width 0.6) (layer "F.Cu") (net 3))
 (segment (start 139.22 108.22) (end 136 105) (width 0.6) (layer "F.Cu") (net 3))
 (segment (start 136 94) (end 135 94) (width 0.6) (layer "F.Cu") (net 3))
 (segment (start 139.22 112) (end 139.22 108.22) (width 0.6) (layer "F.Cu") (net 3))
 (segment (start 146 94) (end 147 95) (width 0.6) (layer "F.Cu") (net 3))
 (segment (start 135.8 112) (end 139.22 112) (width 0.6) (layer "F.Cu") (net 3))
 (segment (start 130 87.45) (end 130 86.5) (width 0.6) (layer "F.Cu") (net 3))
 (segment (start 134 90.75) (end 133.3 90.75) (width 0.6) (layer "F.Cu") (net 3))
 (segment (start 132 95) (end 134 93) (width 0.6) (layer "F.Cu") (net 3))
 (segment (start 147 98) (end 145.19 99.81) (width 0.6) (layer "F.Cu") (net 3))
 (segment (start 147 95) (end 147 98) (width 0.6) (layer "F.Cu") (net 3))
 (segment (start 134 93) (end 134 90.75) (width 0.6) (layer "F.Cu") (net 3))
 (segment (start 132.5 85) (end 132.5 87.25) (width 0.6) (layer "F.Cu") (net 2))
 (segment (start 139 90) (end 142 90) (width 0.6) (layer "F.Cu") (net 2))
 (segment (start 142 90.7) (end 142 90) (width 0.6) (layer "F.Cu") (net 2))
 (segment (start 132.5 87.25) (end 134 88.75) (width 0.6) (layer "F.Cu") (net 2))
 (segment (start 134 88.75) (end 137.75 88.75) (width 0.6) (layer "F.Cu") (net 2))
 (segment (start 132.75 84.75) (end 132.5 85) (width 0.6) (layer "F.Cu") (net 2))
 (segment (start 137.75 88.75) (end 139 90) (width 0.6) (layer "F.Cu") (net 2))
 (segment (start 136.7 84.75) (end 132.75 84.75) (width 0.6) (layer "F.Cu") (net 2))
 (segment (start 132.5 78) (end 132.5 85) (width 0.6) (layer "F.Cu") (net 2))
 (segment (start 133 104) (end 133 112) (width 0.6) (layer "F.Cu") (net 13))
 (segment (start 134.5 80.5) (end 134.5 78) (width 0.6) (layer "F.Cu") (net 6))
 (segment (start 146.425 86.175) (end 150 89.75) (width 0.6) (layer "F.Cu") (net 6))
 (segment (start 138.725794 85.499168) (end 138.725794 84.725794) (width 0.6) (layer "F.Cu") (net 6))
 (segment (start 138.725794 84.725794) (end 134.5 80.5) (width 0.6) (layer "F.Cu") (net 6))
 (segment (start 139.401626 86.175) (end 138.725794 85.499168) (width 0.6) (layer "F.Cu") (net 6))
 (segment (start 146.425 86.175) (end 139.401626 86.175) (width 0.6) (layer "F.Cu") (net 6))
 (segment (start 142.77 97.27) (end 144.22 97.27) (width 0.6) (layer "F.Cu") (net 9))
 (segment (start 167 112) (end 167 96) (width 0.6) (layer "F.Cu") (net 9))
 (segment (start 166 95) (end 161 95) (width 0.6) (layer "F.Cu") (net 9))
 (segment (start 167 96) (end 166 95) (width 0.6) (layer "F.Cu") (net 9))
 (segment (start 140.901 99.139) (end 140.901 103.521) (width 0.6) (layer "F.Cu") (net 9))
 (segment (start 164.648001 114.351999) (end 167 112) (width 0.6) (layer "F.Cu") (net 9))
 (segment (start 151.731999 114.351999) (end 164.648001 114.351999) (width 0.6) (layer "F.Cu") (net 9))
 (segment (start 140.901 99.139) (end 142.77 97.27) (width 0.6) (layer "F.Cu") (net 9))
 (segment (start 149.38 112) (end 151.731999 114.351999) (width 0.6) (layer "F.Cu") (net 9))
 (segment (start 140.901 103.521) (end 149.38 112) (width 0.6) (layer "F.Cu") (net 9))
 (segment (start 157 89) (end 157 93.8) (width 0.6) (layer "F.Cu") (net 14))
 (segment (start 157 93.8) (end 158.2 95) (width 0.6) (layer "F.Cu") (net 14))
 (segment (start 144.22 96) (end 141 96) (width 0.6) (layer "F.Cu") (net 8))
 (segment (start 139 104.16) (end 146.84 112) (width 0.6) (layer "F.Cu") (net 8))
 (segment (start 139 98) (end 139 104.16) (width 0.6) (layer "F.Cu") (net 8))
 (segment (start 141 96) (end 139 98) (width 0.6) (layer "F.Cu") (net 8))
 (segment (start 148 105.54) (end 148 98) (width 0.6) (layer "F.Cu") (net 1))
 (segment (start 151.52 98.54) (end 148.54 98.54) (width 0.6) (layer "F.Cu") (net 1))
 (segment (start 148.54 98.54) (end 148 98) (width 0.6) (layer "F.Cu") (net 1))
 (segment (start 148 98) (end 148 94) (width 0.6) (layer "F.Cu") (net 1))
 (segment (start 154.46 112) (end 148 105.54) (width 0.6) (layer "F.Cu") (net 1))
 (segment (start 148 94) (end 144 90) (width 0.6) (layer "F.Cu") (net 1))
 (segment (start 143.46 98.54) (end 144.22 98.54) (width 0.6) (layer "F.Cu") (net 10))
 (segment (start 151.92 112) (end 142 102.08) (width 0.6) (layer "F.Cu") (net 10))
 (segment (start 142 100) (end 143.46 98.54) (width 0.6) (layer "F.Cu") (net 10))
 (segment (start 142 102.08) (end 142 100) (width 0.6) (layer "F.Cu") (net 10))
 (segment (start 159.54 112) (end 151.52 103.98) (width 0.6) (layer "F.Cu") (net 11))
 (segment (start 151.52 103.98) (end 151.52 99.81) (width 0.6) (layer "F.Cu") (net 11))
 (segment (start 151.52 97.27) (end 152.97 97.27) (width 0.6) (layer "F.Cu") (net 5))
 (segment (start 165 109.3) (end 165 112.725794) (width 0.6) (layer "F.Cu") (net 5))
 (segment (start 165 112.725794) (end 164.274794 113.451) (width 0.6) (layer "F.Cu") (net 5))
 (segment (start 164.274794 113.451) (end 158.451 113.451) (width 0.6) (layer "F.Cu") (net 5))
 (segment (start 151.52 97.27) (end 150.27 97.27) (width 0.6) (layer "F.Cu") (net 5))
 (segment (start 152.97 97.27) (end 165 109.3) (width 0.6) (layer "F.Cu") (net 5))
 (segment (start 158.451 113.451) (end 157 112) (width 0.6) (layer "F.Cu") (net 5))
 (segment (start 150 97) (end 150 91.75) (width 0.6) (layer "F.Cu") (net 5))
 (segment (start 150.27 97.27) (end 150 97) (width 0.6) (layer "F.Cu") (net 5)))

